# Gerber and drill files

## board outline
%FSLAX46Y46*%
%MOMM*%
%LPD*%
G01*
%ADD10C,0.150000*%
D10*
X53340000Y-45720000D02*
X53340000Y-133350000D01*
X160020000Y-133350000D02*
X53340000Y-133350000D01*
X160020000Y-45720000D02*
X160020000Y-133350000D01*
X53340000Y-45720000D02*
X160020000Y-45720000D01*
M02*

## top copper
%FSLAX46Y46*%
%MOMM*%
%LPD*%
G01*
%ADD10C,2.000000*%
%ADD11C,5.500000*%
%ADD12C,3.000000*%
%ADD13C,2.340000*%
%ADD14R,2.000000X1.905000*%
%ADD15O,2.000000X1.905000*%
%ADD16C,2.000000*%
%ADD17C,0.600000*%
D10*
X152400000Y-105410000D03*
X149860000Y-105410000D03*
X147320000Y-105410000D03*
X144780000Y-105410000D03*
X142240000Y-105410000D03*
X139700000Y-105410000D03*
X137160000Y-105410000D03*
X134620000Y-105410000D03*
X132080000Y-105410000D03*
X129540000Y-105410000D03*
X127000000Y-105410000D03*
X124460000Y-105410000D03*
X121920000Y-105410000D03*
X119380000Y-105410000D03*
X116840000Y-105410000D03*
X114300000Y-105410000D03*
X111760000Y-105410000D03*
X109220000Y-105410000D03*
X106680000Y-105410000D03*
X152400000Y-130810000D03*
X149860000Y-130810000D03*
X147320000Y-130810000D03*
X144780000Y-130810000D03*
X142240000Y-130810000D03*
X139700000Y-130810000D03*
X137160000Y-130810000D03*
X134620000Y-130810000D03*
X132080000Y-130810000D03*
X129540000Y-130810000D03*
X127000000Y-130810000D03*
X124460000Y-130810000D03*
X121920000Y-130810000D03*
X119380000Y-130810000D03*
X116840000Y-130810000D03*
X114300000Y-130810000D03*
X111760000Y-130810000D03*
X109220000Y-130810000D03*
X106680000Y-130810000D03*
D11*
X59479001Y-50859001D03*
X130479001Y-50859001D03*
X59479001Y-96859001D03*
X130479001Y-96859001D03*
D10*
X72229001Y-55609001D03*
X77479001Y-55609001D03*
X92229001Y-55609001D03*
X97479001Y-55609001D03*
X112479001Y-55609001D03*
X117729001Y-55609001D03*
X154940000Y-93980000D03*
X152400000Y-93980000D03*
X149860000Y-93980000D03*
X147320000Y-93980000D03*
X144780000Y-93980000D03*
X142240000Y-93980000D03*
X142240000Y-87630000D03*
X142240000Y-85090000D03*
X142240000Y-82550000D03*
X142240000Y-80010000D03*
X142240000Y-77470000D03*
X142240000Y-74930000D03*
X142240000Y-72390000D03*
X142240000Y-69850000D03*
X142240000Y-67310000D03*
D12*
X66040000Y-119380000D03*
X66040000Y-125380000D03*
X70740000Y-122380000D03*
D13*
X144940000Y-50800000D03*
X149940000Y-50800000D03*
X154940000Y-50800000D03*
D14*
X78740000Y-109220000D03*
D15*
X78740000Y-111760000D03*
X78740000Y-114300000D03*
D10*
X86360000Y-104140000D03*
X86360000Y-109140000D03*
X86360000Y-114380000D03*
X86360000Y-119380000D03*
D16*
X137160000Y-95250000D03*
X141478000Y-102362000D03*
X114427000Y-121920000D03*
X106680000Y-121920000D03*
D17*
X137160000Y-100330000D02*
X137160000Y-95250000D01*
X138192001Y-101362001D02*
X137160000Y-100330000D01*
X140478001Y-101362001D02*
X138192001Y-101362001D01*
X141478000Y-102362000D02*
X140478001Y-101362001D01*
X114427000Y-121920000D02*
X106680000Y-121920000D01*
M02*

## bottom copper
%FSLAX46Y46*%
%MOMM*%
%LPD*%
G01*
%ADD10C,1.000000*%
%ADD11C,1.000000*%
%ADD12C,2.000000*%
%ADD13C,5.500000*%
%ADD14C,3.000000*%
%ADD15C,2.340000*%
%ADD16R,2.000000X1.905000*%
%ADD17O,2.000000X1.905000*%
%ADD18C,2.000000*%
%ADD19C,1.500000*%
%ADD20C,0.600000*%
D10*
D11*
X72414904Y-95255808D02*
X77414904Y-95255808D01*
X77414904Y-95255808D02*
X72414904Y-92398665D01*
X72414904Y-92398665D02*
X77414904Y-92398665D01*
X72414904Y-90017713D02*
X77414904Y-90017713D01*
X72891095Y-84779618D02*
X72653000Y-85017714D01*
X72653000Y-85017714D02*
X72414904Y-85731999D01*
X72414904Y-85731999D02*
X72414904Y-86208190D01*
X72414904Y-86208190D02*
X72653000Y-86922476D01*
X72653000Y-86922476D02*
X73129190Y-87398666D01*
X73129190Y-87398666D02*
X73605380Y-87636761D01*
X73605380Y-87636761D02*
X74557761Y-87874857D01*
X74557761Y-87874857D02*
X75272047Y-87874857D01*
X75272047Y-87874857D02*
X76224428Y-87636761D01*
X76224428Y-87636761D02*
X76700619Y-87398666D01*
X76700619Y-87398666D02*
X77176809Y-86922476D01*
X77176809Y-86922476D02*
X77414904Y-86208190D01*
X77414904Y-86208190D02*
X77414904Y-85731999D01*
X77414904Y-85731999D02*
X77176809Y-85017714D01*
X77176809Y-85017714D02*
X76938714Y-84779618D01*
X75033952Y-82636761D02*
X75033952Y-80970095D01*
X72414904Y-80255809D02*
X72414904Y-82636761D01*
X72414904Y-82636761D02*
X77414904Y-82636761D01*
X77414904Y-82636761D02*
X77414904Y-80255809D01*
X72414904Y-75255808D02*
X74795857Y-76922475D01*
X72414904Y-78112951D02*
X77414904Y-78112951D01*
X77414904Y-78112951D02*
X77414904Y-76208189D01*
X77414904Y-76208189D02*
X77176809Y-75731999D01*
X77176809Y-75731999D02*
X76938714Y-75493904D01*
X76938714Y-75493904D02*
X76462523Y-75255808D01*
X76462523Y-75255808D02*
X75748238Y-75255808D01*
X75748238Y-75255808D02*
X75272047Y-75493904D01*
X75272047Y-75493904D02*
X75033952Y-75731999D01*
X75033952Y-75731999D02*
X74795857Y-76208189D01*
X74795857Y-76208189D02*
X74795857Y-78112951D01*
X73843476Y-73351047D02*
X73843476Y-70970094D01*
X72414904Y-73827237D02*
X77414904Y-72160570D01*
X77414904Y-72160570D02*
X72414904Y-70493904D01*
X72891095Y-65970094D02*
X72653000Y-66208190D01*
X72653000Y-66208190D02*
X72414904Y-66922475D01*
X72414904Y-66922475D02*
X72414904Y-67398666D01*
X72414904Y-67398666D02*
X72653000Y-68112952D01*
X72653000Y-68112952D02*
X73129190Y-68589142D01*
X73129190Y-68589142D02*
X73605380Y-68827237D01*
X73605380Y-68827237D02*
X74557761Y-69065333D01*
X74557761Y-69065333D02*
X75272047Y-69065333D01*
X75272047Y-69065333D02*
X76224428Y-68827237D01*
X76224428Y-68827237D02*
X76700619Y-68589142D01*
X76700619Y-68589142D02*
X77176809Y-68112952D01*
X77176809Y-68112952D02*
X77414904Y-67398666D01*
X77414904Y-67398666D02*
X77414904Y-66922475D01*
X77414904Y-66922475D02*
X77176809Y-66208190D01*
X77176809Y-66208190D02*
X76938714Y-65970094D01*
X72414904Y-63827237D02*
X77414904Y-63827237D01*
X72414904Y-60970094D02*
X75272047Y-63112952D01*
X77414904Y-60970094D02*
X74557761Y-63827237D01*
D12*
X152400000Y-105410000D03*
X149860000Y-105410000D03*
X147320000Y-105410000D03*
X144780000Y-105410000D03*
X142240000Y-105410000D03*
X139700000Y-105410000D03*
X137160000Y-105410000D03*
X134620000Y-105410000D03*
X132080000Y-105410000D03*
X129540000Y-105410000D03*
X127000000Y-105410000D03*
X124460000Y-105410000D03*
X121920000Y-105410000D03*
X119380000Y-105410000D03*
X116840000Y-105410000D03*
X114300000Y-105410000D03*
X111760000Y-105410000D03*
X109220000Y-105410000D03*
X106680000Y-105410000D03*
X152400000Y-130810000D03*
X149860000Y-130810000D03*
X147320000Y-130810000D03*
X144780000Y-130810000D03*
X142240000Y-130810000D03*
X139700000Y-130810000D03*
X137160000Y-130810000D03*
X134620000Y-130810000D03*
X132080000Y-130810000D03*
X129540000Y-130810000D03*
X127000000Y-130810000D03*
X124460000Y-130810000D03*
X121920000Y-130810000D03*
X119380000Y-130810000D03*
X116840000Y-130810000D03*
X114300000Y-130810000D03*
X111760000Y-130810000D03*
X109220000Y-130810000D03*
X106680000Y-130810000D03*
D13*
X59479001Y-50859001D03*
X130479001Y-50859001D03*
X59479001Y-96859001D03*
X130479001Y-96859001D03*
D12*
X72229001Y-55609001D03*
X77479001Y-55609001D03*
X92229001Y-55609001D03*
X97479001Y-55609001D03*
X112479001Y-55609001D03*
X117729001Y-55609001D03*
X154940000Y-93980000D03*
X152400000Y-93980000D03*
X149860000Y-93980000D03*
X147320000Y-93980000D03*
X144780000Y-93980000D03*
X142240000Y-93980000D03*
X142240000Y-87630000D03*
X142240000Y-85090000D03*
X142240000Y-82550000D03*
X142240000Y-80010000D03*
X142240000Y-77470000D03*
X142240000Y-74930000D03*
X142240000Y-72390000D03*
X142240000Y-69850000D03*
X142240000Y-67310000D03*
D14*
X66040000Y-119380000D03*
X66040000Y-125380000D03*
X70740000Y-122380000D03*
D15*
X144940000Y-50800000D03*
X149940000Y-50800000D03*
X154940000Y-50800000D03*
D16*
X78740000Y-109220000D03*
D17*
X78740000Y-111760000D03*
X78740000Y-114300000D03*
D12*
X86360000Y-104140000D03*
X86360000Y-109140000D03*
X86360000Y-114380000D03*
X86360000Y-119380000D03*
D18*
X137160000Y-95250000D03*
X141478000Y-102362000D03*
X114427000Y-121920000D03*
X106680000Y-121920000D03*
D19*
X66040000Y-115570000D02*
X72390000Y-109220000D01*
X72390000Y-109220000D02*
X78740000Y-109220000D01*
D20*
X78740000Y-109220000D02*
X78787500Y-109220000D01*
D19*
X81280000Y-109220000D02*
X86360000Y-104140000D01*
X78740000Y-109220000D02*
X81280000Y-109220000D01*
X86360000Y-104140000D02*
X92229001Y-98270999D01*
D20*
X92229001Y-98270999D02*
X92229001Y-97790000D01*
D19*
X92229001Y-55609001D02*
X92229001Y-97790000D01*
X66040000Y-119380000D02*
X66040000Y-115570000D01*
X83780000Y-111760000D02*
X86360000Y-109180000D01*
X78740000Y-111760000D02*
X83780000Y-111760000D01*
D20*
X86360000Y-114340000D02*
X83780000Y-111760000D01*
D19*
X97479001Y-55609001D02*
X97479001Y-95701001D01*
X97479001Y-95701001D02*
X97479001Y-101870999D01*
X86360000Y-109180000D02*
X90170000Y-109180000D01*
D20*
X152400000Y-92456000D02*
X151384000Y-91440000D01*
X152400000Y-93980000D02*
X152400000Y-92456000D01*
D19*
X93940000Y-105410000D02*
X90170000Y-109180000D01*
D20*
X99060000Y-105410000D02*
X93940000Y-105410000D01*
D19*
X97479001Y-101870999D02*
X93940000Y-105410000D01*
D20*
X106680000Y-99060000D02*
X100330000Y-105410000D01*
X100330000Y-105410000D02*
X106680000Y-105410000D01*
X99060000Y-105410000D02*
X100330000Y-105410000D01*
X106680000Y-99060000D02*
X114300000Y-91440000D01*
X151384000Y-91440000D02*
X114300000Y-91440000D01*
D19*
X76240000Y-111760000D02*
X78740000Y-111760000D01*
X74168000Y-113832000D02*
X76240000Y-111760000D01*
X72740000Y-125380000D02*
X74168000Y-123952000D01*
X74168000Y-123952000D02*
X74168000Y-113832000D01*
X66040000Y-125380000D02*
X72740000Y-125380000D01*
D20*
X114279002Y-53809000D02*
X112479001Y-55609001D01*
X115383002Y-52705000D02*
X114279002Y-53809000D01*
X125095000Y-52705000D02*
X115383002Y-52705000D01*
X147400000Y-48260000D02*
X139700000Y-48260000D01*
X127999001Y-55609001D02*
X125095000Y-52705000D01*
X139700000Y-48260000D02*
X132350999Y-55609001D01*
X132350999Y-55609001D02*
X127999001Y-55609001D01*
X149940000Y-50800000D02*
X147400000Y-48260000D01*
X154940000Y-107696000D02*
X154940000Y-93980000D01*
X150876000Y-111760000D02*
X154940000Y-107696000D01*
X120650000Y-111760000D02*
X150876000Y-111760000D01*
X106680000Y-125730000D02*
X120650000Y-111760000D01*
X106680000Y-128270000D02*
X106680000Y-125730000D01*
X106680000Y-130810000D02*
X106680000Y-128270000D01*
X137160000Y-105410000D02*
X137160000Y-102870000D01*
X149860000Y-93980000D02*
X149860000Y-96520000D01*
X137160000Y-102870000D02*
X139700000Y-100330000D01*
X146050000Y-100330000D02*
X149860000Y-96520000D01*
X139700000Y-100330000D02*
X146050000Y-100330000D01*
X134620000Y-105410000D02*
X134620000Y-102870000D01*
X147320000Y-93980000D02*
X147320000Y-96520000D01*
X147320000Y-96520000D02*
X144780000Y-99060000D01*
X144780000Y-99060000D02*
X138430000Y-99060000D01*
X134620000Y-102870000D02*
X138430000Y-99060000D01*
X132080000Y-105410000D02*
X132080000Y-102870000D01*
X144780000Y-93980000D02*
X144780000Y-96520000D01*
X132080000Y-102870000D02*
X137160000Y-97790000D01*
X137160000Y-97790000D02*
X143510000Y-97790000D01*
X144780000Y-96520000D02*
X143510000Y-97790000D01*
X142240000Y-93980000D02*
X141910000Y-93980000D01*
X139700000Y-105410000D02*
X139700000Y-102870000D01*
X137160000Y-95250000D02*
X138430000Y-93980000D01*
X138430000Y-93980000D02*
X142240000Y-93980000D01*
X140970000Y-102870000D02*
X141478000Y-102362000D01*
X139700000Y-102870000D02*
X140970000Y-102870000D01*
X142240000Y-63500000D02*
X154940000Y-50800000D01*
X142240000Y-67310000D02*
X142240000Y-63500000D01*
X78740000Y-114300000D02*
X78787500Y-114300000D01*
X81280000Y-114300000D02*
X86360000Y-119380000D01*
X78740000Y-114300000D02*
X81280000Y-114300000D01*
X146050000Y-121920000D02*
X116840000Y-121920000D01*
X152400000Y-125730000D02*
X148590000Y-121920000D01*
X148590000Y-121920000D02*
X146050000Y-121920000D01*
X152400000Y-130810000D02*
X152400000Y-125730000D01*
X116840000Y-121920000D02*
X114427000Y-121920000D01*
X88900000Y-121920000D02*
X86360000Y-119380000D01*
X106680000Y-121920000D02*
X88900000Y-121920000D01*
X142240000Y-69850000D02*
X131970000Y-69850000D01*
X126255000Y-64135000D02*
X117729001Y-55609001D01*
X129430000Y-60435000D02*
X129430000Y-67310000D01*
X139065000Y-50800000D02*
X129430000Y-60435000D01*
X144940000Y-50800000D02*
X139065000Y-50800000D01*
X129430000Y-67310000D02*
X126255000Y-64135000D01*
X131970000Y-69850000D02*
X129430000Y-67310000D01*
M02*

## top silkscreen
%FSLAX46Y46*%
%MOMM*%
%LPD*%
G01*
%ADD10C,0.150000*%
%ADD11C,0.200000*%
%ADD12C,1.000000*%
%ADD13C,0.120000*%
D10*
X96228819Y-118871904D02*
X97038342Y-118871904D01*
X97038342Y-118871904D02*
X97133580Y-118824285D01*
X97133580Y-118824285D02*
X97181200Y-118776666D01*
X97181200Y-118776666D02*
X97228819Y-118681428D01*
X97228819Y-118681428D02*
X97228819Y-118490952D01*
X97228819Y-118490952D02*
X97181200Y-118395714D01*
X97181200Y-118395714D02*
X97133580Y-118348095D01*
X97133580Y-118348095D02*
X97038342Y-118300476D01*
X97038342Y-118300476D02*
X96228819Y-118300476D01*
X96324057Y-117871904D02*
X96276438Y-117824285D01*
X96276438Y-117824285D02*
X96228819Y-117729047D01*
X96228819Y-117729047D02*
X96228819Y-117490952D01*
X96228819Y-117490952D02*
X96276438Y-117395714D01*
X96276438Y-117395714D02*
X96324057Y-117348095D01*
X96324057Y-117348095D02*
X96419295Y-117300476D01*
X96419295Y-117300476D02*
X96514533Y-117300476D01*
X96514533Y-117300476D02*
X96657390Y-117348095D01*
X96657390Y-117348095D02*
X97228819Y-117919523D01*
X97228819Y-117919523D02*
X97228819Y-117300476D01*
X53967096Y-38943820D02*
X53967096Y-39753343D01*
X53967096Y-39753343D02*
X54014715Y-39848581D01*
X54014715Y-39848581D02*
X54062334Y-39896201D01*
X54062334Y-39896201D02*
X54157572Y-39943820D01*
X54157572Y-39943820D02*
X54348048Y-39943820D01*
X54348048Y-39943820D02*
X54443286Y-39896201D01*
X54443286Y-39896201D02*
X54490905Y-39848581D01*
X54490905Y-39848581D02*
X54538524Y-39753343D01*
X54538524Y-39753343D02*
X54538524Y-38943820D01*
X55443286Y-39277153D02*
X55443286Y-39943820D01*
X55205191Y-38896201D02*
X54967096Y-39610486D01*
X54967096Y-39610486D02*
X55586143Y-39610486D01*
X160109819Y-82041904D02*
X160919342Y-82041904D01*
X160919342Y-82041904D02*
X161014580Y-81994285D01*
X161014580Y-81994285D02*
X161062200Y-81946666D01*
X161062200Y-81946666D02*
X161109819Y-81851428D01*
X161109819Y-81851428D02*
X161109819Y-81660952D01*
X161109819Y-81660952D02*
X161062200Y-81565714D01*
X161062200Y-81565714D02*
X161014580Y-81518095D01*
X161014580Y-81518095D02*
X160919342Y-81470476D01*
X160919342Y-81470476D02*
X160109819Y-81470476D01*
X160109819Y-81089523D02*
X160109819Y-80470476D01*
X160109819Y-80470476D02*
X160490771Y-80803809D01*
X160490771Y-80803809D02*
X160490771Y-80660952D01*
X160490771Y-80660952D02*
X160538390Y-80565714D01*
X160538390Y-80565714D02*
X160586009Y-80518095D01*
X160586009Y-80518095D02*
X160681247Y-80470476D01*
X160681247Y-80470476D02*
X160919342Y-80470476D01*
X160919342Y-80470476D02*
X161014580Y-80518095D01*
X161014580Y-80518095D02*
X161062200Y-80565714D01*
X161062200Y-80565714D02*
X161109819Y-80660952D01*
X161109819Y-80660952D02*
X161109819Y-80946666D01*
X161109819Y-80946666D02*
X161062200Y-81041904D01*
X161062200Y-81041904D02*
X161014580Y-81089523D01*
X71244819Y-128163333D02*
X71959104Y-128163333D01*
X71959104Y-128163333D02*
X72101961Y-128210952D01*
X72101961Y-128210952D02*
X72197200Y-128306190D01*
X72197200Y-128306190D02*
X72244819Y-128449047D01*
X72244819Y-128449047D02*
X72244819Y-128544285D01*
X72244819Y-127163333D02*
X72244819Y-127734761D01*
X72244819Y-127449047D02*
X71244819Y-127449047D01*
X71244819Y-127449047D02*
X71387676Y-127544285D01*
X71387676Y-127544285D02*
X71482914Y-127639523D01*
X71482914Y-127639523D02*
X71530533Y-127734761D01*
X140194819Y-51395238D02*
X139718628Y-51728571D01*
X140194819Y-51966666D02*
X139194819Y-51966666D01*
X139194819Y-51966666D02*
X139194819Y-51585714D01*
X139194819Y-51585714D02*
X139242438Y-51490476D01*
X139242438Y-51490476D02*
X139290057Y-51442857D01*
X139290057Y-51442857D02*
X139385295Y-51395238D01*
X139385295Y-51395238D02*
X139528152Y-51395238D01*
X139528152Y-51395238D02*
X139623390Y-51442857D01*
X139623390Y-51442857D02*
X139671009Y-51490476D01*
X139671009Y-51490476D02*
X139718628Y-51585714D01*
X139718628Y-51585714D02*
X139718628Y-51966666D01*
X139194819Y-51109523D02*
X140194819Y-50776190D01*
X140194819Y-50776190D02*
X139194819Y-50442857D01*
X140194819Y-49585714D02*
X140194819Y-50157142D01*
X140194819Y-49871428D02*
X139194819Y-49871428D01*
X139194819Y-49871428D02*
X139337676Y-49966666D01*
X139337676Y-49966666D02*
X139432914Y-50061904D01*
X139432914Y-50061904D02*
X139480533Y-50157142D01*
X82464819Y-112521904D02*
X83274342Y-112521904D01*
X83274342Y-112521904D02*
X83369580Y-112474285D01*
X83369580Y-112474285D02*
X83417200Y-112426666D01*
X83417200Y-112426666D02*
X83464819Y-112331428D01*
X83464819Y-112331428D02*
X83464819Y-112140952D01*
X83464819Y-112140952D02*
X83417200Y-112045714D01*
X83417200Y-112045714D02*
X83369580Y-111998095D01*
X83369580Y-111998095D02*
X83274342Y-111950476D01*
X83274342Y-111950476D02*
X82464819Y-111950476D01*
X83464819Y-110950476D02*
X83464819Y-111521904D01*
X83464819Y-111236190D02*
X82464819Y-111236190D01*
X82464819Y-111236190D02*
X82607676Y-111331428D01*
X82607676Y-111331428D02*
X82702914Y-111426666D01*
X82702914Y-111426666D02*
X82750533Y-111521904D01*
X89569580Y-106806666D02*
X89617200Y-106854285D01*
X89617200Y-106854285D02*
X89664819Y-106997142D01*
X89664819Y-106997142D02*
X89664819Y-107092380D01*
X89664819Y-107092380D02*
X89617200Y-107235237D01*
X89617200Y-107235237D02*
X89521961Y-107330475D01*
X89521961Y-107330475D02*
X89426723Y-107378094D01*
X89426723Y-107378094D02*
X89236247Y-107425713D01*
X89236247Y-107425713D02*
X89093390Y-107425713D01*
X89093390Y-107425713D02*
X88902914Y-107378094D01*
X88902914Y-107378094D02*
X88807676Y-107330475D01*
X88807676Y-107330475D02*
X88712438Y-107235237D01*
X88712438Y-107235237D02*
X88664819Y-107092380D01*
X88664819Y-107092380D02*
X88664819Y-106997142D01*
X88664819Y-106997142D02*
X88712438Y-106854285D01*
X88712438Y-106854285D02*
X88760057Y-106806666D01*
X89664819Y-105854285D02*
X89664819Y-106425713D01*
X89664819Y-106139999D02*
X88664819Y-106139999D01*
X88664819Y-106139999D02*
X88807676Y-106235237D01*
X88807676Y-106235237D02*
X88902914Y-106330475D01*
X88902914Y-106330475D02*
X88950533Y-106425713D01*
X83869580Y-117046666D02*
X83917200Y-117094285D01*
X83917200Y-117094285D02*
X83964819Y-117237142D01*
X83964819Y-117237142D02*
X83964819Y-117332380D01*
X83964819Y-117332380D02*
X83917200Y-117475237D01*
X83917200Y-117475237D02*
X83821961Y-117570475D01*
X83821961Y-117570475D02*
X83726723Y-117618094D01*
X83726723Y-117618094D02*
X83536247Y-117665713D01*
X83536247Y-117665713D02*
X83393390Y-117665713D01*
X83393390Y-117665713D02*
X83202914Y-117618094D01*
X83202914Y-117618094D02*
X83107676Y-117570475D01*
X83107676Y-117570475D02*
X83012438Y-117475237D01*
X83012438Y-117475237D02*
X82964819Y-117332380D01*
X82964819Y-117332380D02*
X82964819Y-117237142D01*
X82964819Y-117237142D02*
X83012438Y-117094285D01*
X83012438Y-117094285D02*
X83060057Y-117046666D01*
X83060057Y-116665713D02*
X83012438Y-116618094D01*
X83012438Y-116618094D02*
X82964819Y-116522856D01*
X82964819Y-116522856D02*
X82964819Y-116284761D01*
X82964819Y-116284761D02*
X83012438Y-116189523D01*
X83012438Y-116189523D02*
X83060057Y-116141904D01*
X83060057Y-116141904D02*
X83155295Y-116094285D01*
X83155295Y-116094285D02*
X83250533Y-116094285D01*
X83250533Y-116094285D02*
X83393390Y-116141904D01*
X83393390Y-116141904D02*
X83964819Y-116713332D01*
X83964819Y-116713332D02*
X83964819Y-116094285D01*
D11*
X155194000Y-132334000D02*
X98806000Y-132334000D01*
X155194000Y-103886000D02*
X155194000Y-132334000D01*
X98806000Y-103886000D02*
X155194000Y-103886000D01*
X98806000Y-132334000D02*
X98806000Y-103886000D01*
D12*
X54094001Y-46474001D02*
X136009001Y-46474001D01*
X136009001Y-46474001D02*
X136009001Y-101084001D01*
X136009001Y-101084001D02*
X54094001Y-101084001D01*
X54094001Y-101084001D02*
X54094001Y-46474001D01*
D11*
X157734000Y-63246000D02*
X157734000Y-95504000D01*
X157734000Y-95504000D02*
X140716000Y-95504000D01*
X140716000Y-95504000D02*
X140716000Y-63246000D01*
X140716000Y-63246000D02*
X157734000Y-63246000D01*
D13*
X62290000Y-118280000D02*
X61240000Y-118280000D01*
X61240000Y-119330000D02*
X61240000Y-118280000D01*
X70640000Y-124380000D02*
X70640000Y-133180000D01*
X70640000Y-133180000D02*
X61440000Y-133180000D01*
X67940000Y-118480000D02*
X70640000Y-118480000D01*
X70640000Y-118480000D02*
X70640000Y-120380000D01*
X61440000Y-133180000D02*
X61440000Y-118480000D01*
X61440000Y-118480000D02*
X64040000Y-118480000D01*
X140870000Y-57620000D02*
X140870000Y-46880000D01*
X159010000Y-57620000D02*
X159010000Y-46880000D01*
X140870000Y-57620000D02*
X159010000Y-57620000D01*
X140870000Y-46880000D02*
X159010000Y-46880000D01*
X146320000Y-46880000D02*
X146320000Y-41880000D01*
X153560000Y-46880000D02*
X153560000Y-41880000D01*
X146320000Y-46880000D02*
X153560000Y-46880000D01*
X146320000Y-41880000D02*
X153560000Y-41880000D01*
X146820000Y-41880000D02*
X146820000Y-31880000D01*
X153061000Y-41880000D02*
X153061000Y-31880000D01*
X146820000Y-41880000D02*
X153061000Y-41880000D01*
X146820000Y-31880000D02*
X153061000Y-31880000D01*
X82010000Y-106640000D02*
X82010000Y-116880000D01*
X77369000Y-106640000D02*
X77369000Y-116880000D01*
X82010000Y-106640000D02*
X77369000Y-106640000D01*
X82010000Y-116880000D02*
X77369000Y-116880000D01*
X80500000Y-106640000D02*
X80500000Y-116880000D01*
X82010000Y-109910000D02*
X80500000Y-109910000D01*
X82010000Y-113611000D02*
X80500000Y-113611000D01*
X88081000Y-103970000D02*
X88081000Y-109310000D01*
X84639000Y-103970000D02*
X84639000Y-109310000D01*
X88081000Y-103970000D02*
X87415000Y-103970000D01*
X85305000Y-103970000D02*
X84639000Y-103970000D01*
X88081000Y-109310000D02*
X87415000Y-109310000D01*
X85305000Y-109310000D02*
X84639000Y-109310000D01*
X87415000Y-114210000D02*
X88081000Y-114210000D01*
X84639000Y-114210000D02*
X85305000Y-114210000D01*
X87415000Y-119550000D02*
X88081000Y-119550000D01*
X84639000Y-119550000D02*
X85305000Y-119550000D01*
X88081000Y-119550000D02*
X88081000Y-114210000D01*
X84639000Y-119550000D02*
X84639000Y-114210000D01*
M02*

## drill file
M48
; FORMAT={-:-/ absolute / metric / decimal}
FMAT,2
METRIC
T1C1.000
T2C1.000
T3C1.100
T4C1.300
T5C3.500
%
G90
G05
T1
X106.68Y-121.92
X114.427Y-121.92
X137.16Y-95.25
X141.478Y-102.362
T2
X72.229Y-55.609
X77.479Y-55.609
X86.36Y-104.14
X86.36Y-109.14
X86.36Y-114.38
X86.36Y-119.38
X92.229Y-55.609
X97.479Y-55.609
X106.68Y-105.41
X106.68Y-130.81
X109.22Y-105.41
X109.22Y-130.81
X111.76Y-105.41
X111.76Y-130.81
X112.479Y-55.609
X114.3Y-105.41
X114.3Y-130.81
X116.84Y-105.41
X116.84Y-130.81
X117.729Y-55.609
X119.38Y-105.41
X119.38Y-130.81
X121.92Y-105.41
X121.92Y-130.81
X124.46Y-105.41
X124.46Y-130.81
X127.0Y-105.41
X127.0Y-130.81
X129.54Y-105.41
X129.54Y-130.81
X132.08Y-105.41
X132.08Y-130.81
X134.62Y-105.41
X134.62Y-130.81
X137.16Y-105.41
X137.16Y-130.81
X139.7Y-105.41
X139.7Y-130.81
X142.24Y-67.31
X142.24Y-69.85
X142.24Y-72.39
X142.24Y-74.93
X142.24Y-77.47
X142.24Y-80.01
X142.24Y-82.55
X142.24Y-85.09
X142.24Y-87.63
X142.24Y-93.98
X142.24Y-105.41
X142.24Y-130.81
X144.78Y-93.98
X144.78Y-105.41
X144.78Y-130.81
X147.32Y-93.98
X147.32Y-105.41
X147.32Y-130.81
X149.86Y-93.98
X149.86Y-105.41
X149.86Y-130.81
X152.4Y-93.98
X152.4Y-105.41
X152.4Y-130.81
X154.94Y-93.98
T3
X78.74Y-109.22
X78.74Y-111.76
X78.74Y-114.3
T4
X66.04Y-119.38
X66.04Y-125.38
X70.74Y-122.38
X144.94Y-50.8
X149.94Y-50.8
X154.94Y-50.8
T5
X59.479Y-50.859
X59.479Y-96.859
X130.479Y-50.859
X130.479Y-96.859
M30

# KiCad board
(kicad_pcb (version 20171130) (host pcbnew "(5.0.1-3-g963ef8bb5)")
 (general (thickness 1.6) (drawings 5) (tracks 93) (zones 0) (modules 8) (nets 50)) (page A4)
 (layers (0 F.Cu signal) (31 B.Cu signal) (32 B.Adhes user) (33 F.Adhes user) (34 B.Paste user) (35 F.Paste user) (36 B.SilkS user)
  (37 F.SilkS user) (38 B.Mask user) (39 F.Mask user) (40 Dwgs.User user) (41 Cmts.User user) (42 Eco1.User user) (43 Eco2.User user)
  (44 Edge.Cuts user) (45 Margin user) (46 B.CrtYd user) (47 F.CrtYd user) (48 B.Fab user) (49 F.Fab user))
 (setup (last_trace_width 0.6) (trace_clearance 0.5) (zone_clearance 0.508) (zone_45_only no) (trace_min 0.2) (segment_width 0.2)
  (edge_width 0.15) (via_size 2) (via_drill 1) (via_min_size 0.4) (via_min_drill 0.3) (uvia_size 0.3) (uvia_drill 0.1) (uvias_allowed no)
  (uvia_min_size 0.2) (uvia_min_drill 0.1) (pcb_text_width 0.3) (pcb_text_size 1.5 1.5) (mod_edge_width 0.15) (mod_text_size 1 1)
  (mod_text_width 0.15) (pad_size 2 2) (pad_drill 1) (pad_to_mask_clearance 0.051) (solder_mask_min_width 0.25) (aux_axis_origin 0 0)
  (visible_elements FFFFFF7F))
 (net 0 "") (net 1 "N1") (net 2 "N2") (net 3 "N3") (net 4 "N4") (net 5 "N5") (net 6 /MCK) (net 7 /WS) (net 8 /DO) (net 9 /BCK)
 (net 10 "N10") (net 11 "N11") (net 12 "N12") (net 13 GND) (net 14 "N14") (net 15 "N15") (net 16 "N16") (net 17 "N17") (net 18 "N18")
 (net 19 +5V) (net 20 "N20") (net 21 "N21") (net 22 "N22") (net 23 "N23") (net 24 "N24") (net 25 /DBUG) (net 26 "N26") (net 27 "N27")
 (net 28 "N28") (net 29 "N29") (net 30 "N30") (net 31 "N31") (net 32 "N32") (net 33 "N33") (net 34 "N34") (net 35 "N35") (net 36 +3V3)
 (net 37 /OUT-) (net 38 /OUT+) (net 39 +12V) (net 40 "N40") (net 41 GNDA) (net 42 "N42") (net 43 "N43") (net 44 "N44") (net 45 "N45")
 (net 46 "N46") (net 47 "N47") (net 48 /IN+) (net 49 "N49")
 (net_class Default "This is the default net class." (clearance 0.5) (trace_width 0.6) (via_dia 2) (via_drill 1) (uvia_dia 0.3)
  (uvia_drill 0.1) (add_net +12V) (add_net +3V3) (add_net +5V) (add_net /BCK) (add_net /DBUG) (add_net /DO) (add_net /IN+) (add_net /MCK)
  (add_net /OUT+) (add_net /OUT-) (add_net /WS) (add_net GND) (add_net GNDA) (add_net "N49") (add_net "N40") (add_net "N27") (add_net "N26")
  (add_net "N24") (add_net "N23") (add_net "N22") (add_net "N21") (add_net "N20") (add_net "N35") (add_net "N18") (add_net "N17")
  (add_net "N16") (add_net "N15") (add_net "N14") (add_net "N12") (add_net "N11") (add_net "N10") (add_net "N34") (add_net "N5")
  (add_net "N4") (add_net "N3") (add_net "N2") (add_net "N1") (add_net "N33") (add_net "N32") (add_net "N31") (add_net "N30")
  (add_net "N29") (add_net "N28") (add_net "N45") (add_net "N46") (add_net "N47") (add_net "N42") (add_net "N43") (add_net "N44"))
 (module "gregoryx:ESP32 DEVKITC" (layer F.Cu) (at 104.14 118.11 90)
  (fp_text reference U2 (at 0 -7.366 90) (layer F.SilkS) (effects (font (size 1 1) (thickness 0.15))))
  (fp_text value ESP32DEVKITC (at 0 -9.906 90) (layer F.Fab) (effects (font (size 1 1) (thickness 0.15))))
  (fp_line (start -14.224 51.054) (end -14.224 -5.334) (layer F.SilkS) (width 0.2))
  (fp_line (start 14.224 51.054) (end -14.224 51.054) (layer F.SilkS) (width 0.2))
  (fp_line (start 14.224 -5.334) (end 14.224 51.054) (layer F.SilkS) (width 0.2))
  (fp_line (start -14.224 -5.334) (end 14.224 -5.334) (layer F.SilkS) (width 0.2))
  (pad 38 thru_hole circle (at 12.7 48.26 90) (size 2 2) (drill 1) (layers *.Cu *.Mask) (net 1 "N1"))
  (pad 37 thru_hole circle (at 12.7 45.72 90) (size 2 2) (drill 1) (layers *.Cu *.Mask) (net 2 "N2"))
  (pad 36 thru_hole circle (at 12.7 43.18 90) (size 2 2) (drill 1) (layers *.Cu *.Mask) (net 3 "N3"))
  (pad 35 thru_hole circle (at 12.7 40.64 90) (size 2 2) (drill 1) (layers *.Cu *.Mask) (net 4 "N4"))
  (pad 34 thru_hole circle (at 12.7 38.1 90) (size 2 2) (drill 1) (layers *.Cu *.Mask) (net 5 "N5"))
  (pad 33 thru_hole circle (at 12.7 35.56 90) (size 2 2) (drill 1) (layers *.Cu *.Mask) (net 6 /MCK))
  (pad 32 thru_hole circle (at 12.7 33.02 90) (size 2 2) (drill 1) (layers *.Cu *.Mask) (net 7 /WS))
  (pad 31 thru_hole circle (at 12.7 30.48 90) (size 2 2) (drill 1) (layers *.Cu *.Mask) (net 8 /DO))
  (pad 30 thru_hole circle (at 12.7 27.94 90) (size 2 2) (drill 1) (layers *.Cu *.Mask) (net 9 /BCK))
  (pad 29 thru_hole circle (at 12.7 25.4 90) (size 2 2) (drill 1) (layers *.Cu *.Mask) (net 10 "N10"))
  (pad 28 thru_hole circle (at 12.7 22.86 90) (size 2 2) (drill 1) (layers *.Cu *.Mask) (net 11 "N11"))
  (pad 27 thru_hole circle (at 12.7 20.32 90) (size 2 2) (drill 1) (layers *.Cu *.Mask) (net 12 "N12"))
  (pad 26 thru_hole circle (at 12.7 17.78 90) (size 2 2) (drill 1) (layers *.Cu *.Mask) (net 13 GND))
  (pad 25 thru_hole circle (at 12.7 15.24 90) (size 2 2) (drill 1) (layers *.Cu *.Mask) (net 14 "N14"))
  (pad 24 thru_hole circle (at 12.7 12.7 90) (size 2 2) (drill 1) (layers *.Cu *.Mask) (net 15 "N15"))
  (pad 23 thru_hole circle (at 12.7 10.16 90) (size 2 2) (drill 1) (layers *.Cu *.Mask) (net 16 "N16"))
  (pad 22 thru_hole circle (at 12.7 7.62 90) (size 2 2) (drill 1) (layers *.Cu *.Mask) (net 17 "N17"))
  (pad 21 thru_hole circle (at 12.7 5.08 90) (size 2 2) (drill 1) (layers *.Cu *.Mask) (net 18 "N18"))
  (pad 20 thru_hole circle (at 12.7 2.54 90) (size 2 2) (drill 1) (layers *.Cu *.Mask) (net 13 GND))
  (pad 19 thru_hole circle (at -12.7 48.26 90) (size 2 2) (drill 1) (layers *.Cu *.Mask) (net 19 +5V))
  (pad 18 thru_hole circle (at -12.7 45.72 90) (size 2 2) (drill 1) (layers *.Cu *.Mask) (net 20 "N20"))
  (pad 17 thru_hole circle (at -12.7 43.18 90) (size 2 2) (drill 1) (layers *.Cu *.Mask) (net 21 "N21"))
  (pad 16 thru_hole circle (at -12.7 40.64 90) (size 2 2) (drill 1) (layers *.Cu *.Mask) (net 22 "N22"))
  (pad 15 thru_hole circle (at -12.7 38.1 90) (size 2 2) (drill 1) (layers *.Cu *.Mask) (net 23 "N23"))
  (pad 14 thru_hole circle (at -12.7 35.56 90) (size 2 2) (drill 1) (layers *.Cu *.Mask) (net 13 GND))
  (pad 13 thru_hole circle (at -12.7 33.02 90) (size 2 2) (drill 1) (layers *.Cu *.Mask) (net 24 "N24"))
  (pad 12 thru_hole circle (at -12.7 30.48 90) (size 2 2) (drill 1) (layers *.Cu *.Mask) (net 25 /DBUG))
  (pad 11 thru_hole circle (at -12.7 27.94 90) (size 2 2) (drill 1) (layers *.Cu *.Mask) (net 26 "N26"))
  (pad 10 thru_hole circle (at -12.7 25.4 90) (size 2 2) (drill 1) (layers *.Cu *.Mask) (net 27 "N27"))
  (pad 9 thru_hole circle (at -12.7 22.86 90) (size 2 2) (drill 1) (layers *.Cu *.Mask) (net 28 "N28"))
  (pad 8 thru_hole circle (at -12.7 20.32 90) (size 2 2) (drill 1) (layers *.Cu *.Mask) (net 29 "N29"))
  (pad 7 thru_hole circle (at -12.7 17.78 90) (size 2 2) (drill 1) (layers *.Cu *.Mask) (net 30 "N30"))
  (pad 6 thru_hole circle (at -12.7 15.24 90) (size 2 2) (drill 1) (layers *.Cu *.Mask) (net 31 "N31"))
  (pad 5 thru_hole circle (at -12.7 12.7 90) (size 2 2) (drill 1) (layers *.Cu *.Mask) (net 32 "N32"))
  (pad 4 thru_hole circle (at -12.7 10.16 90) (size 2 2) (drill 1) (layers *.Cu *.Mask) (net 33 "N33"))
  (pad 3 thru_hole circle (at -12.7 7.62 90) (size 2 2) (drill 1) (layers *.Cu *.Mask) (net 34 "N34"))
  (pad 2 thru_hole circle (at -12.7 5.08 90) (size 2 2) (drill 1) (layers *.Cu *.Mask) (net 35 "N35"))
  (pad 1 thru_hole circle (at -12.7 2.54 90) (size 2 2) (drill 1) (layers *.Cu *.Mask) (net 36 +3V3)))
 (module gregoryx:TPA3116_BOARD (layer F.Cu) (at 54.729001 47.109001)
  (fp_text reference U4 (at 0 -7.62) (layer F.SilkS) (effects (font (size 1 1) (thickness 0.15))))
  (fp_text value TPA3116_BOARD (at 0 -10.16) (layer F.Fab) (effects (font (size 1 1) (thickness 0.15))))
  (fp_line (start -0.635 -0.635) (end 81.28 -0.635) (layer F.SilkS) (width 1))
  (fp_line (start 81.28 -0.635) (end 81.28 53.975) (layer F.SilkS) (width 1))
  (fp_line (start 81.28 53.975) (end -0.635 53.975) (layer F.SilkS) (width 1))
  (fp_line (start -0.635 53.975) (end -0.635 -0.635) (layer F.SilkS) (width 1))
  (pad "" thru_hole circle (at 4.75 3.75) (size 5.5 5.5) (drill 3.5) (layers *.Cu *.Mask))
  (pad "" thru_hole circle (at 75.75 3.75) (size 5.5 5.5) (drill 3.5) (layers *.Cu *.Mask))
  (pad "" thru_hole circle (at 4.75 49.75) (size 5.5 5.5) (drill 3.5) (layers *.Cu *.Mask))
  (pad "" thru_hole circle (at 75.75 49.75) (size 5.5 5.5) (drill 3.5) (layers *.Cu *.Mask))
  (pad 6 thru_hole circle (at 17.5 8.5) (size 2 2) (drill 1) (layers *.Cu *.Mask) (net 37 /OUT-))
  (pad 5 thru_hole circle (at 22.75 8.5) (size 2 2) (drill 1) (layers *.Cu *.Mask) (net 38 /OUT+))
  (pad 4 thru_hole circle (at 37.5 8.5) (size 2 2) (drill 1) (layers *.Cu *.Mask) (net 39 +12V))
  (pad 3 thru_hole circle (at 42.75 8.5) (size 2 2) (drill 1) (layers *.Cu *.Mask) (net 13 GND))
  (pad 2 thru_hole circle (at 57.75 8.5) (size 2 2) (drill 1) (layers *.Cu *.Mask) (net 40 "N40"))
  (pad 1 thru_hole circle (at 63 8.5) (size 2 2) (drill 1) (layers *.Cu *.Mask) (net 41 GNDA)))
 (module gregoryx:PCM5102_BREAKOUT (layer F.Cu) (at 157.48 81.28 270)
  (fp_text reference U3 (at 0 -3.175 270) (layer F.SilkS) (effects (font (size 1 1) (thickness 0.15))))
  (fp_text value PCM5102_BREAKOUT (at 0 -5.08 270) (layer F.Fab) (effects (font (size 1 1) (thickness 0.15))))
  (fp_line (start -18.034 -0.254) (end 14.224 -0.254) (layer F.SilkS) (width 0.2))
  (fp_line (start 14.224 -0.254) (end 14.224 16.764) (layer F.SilkS) (width 0.2))
  (fp_line (start 14.224 16.764) (end -18.034 16.764) (layer F.SilkS) (width 0.2))
  (fp_line (start -18.034 16.764) (end -18.034 -0.254) (layer F.SilkS) (width 0.2))
  (pad 1 thru_hole circle (at 12.7 2.54 270) (size 2 2) (drill 1) (layers *.Cu *.Mask) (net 36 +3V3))
  (pad 2 thru_hole circle (at 12.7 5.08 270) (size 2 2) (drill 1) (layers *.Cu *.Mask) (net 13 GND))
  (pad 3 thru_hole circle (at 12.7 7.62 270) (size 2 2) (drill 1) (layers *.Cu *.Mask) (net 7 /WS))
  (pad 4 thru_hole circle (at 12.7 10.16 270) (size 2 2) (drill 1) (layers *.Cu *.Mask) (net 8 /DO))
  (pad 5 thru_hole circle (at 12.7 12.7 270) (size 2 2) (drill 1) (layers *.Cu *.Mask) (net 9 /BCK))
  (pad 6 thru_hole circle (at 12.7 15.24 270) (size 2 2) (drill 1) (layers *.Cu *.Mask) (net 6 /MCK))
  (pad 7 thru_hole circle (at 6.35 15.24 270) (size 2 2) (drill 1) (layers *.Cu *.Mask) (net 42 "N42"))
  (pad 8 thru_hole circle (at 3.81 15.24 270) (size 2 2) (drill 1) (layers *.Cu *.Mask) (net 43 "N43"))
  (pad 9 thru_hole circle (at 1.27 15.24 270) (size 2 2) (drill 1) (layers *.Cu *.Mask) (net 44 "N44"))
  (pad 10 thru_hole circle (at -1.27 15.24 270) (size 2 2) (drill 1) (layers *.Cu *.Mask) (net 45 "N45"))
  (pad "" thru_hole circle (at -3.81 15.24 270) (size 2 2) (drill 1) (layers *.Cu *.Mask))
  (pad 11 thru_hole circle (at -6.35 15.24 270) (size 2 2) (drill 1) (layers *.Cu *.Mask) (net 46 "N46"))
  (pad 12 thru_hole circle (at -8.89 15.24 270) (size 2 2) (drill 1) (layers *.Cu *.Mask) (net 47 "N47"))
  (pad 13 thru_hole circle (at -11.43 15.24 270) (size 2 2) (drill 1) (layers *.Cu *.Mask) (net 41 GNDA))
  (pad 14 thru_hole circle (at -13.97 15.24 270) (size 2 2) (drill 1) (layers *.Cu *.Mask) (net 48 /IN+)))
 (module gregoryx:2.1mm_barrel (layer F.Cu) (at 66.04 119.38 90)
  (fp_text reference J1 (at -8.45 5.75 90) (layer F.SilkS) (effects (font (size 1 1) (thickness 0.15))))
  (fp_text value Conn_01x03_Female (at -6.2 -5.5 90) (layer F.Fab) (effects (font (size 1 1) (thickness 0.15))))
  (fp_line (start 1.1 -3.75) (end 1.1 -4.8) (layer F.SilkS) (width 0.12))
  (fp_line (start 0.05 -4.8) (end 1.1 -4.8) (layer F.SilkS) (width 0.12))
  (fp_line (start -5 4.6) (end -13.8 4.6) (layer F.SilkS) (width 0.12))
  (fp_line (start -13.8 4.6) (end -13.8 -4.6) (layer F.SilkS) (width 0.12))
  (fp_line (start 0.9 1.9) (end 0.9 4.6) (layer F.SilkS) (width 0.12))
  (fp_line (start 0.9 4.6) (end -1 4.6) (layer F.SilkS) (width 0.12))
  (fp_line (start -13.8 -4.6) (end 0.9 -4.6) (layer F.SilkS) (width 0.12))
  (fp_line (start 0.9 -4.6) (end 0.9 -2) (layer F.SilkS) (width 0.12))
  (pad 1 thru_hole circle (at 0 0 90) (size 3 3) (drill 1.3) (layers *.Cu *.Mask) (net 39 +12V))
  (pad 2 thru_hole circle (at -6 0 90) (size 3 3) (drill 1.3) (layers *.Cu *.Mask) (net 13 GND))
  (pad 3 thru_hole circle (at -3 4.7 90) (size 3 3) (drill 1.3) (layers *.Cu *.Mask) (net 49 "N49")))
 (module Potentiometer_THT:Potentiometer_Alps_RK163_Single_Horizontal (layer F.Cu) (at 154.94 50.8 90)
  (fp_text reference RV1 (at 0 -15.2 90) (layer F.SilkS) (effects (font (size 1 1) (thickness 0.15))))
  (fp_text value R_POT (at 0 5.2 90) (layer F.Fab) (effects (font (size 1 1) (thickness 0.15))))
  (fp_line (start -6.82 -14.07) (end 3.92 -14.07) (layer F.SilkS) (width 0.12))
  (fp_line (start -6.82 4.07) (end 3.92 4.07) (layer F.SilkS) (width 0.12))
  (fp_line (start -6.82 -14.07) (end -6.82 4.07) (layer F.SilkS) (width 0.12))
  (fp_line (start 3.92 -14.07) (end 3.92 4.07) (layer F.SilkS) (width 0.12))
  (fp_line (start 3.92 -8.62) (end 8.92 -8.62) (layer F.SilkS) (width 0.12))
  (fp_line (start 3.92 -1.38) (end 8.92 -1.38) (layer F.SilkS) (width 0.12))
  (fp_line (start 3.92 -8.62) (end 3.92 -1.38) (layer F.SilkS) (width 0.12))
  (fp_line (start 8.92 -8.62) (end 8.92 -1.38) (layer F.SilkS) (width 0.12))
  (fp_line (start 8.92 -8.12) (end 18.92 -8.12) (layer F.SilkS) (width 0.12))
  (fp_line (start 8.92 -1.879) (end 18.92 -1.879) (layer F.SilkS) (width 0.12))
  (fp_line (start 8.92 -8.12) (end 8.92 -1.879) (layer F.SilkS) (width 0.12))
  (fp_line (start 18.92 -8.12) (end 18.92 -1.879) (layer F.SilkS) (width 0.12))
  (pad 3 thru_hole circle (at 0 -10 90) (size 2.34 2.34) (drill 1.3) (layers *.Cu *.Mask) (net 41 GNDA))
  (pad 2 thru_hole circle (at 0 -5 90) (size 2.34 2.34) (drill 1.3) (layers *.Cu *.Mask) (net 40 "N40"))
  (pad 1 thru_hole circle (at 0 0 90) (size 2.34 2.34) (drill 1.3) (layers *.Cu *.Mask) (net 48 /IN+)))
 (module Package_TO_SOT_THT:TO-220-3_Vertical (layer F.Cu) (at 78.74 109.22 270)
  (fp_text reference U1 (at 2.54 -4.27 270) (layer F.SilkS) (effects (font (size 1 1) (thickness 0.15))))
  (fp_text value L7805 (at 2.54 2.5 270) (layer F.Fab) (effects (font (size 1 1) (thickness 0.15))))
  (fp_line (start -2.58 -3.27) (end 7.66 -3.27) (layer F.SilkS) (width 0.12))
  (fp_line (start -2.58 1.371) (end 7.66 1.371) (layer F.SilkS) (width 0.12))
  (fp_line (start -2.58 -3.27) (end -2.58 1.371) (layer F.SilkS) (width 0.12))
  (fp_line (start 7.66 -3.27) (end 7.66 1.371) (layer F.SilkS) (width 0.12))
  (fp_line (start -2.58 -1.76) (end 7.66 -1.76) (layer F.SilkS) (width 0.12))
  (fp_line (start 0.69 -3.27) (end 0.69 -1.76) (layer F.SilkS) (width 0.12))
  (fp_line (start 4.391 -3.27) (end 4.391 -1.76) (layer F.SilkS) (width 0.12))
  (pad 1 thru_hole rect (at 0 0 270) (size 1.905 2) (drill 1.1) (layers *.Cu *.Mask) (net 39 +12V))
  (pad 2 thru_hole oval (at 2.54 0 270) (size 1.905 2) (drill 1.1) (layers *.Cu *.Mask) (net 13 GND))
  (pad 3 thru_hole oval (at 5.08 0 270) (size 1.905 2) (drill 1.1) (layers *.Cu *.Mask) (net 19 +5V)))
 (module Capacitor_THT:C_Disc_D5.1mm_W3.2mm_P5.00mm (layer F.Cu) (at 86.36 104.14 270)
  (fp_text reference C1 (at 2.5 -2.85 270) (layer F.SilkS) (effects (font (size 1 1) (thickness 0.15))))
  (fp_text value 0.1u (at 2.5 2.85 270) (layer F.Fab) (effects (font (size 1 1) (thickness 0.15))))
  (fp_line (start -0.17 -1.721) (end 5.17 -1.721) (layer F.SilkS) (width 0.12))
  (fp_line (start -0.17 1.721) (end 5.17 1.721) (layer F.SilkS) (width 0.12))
  (fp_line (start -0.17 -1.721) (end -0.17 -1.055) (layer F.SilkS) (width 0.12))
  (fp_line (start -0.17 1.055) (end -0.17 1.721) (layer F.SilkS) (width 0.12))
  (fp_line (start 5.17 -1.721) (end 5.17 -1.055) (layer F.SilkS) (width 0.12))
  (fp_line (start 5.17 1.055) (end 5.17 1.721) (layer F.SilkS) (width 0.12))
  (pad 1 thru_hole circle (at 0 0 270) (size 2 2) (drill 1) (layers *.Cu *.Mask) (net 39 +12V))
  (pad 2 thru_hole circle (at 5 0 270) (size 2 2) (drill 1) (layers *.Cu *.Mask) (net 13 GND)))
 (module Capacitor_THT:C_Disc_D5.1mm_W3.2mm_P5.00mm (layer F.Cu) (at 86.36 119.38 90)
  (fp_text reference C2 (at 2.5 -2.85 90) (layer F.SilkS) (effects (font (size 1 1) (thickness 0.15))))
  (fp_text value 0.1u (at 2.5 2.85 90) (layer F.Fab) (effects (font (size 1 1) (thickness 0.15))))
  (fp_line (start 5.17 1.055) (end 5.17 1.721) (layer F.SilkS) (width 0.12))
  (fp_line (start 5.17 -1.721) (end 5.17 -1.055) (layer F.SilkS) (width 0.12))
  (fp_line (start -0.17 1.055) (end -0.17 1.721) (layer F.SilkS) (width 0.12))
  (fp_line (start -0.17 -1.721) (end -0.17 -1.055) (layer F.SilkS) (width 0.12))
  (fp_line (start -0.17 1.721) (end 5.17 1.721) (layer F.SilkS) (width 0.12))
  (fp_line (start -0.17 -1.721) (end 5.17 -1.721) (layer F.SilkS) (width 0.12))
  (pad 2 thru_hole circle (at 5 0 90) (size 2 2) (drill 1) (layers *.Cu *.Mask) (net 13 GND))
  (pad 1 thru_hole circle (at 0 0 90) (size 2 2) (drill 1) (layers *.Cu *.Mask) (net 19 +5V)))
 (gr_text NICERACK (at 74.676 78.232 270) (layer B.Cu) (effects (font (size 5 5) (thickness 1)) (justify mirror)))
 (gr_line (start 53.34 45.72) (end 53.34 133.35) (layer Edge.Cuts) (width 0.15))
 (gr_line (start 160.02 133.35) (end 53.34 133.35) (layer Edge.Cuts) (width 0.15))
 (gr_line (start 160.02 45.72) (end 160.02 133.35) (layer Edge.Cuts) (width 0.15))
 (gr_line (start 53.34 45.72) (end 160.02 45.72) (layer Edge.Cuts) (width 0.15))
 (segment (start 66.04 115.57) (end 72.39 109.22) (width 1.5) (layer B.Cu) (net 39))
 (segment (start 72.39 109.22) (end 78.74 109.22) (width 1.5) (layer B.Cu) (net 39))
 (segment (start 78.74 109.22) (end 78.7875 109.22) (width 0.6) (layer B.Cu) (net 39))
 (segment (start 81.28 109.22) (end 86.36 104.14) (width 1.5) (layer B.Cu) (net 39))
 (segment (start 78.74 109.22) (end 81.28 109.22) (width 1.5) (layer B.Cu) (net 39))
 (segment (start 86.36 104.14) (end 92.229001 98.270999) (width 1.5) (layer B.Cu) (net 39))
 (segment (start 92.229001 98.270999) (end 92.229001 97.79) (width 0.6) (layer B.Cu) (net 39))
 (segment (start 92.229001 55.609001) (end 92.229001 97.79) (width 1.5) (layer B.Cu) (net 39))
 (segment (start 66.04 119.38) (end 66.04 115.57) (width 1.5) (layer B.Cu) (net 39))
 (segment (start 83.78 111.76) (end 86.36 109.18) (width 1.5) (layer B.Cu) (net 13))
 (segment (start 78.74 111.76) (end 83.78 111.76) (width 1.5) (layer B.Cu) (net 13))
 (segment (start 86.36 114.34) (end 83.78 111.76) (width 0.6) (layer B.Cu) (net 13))
 (segment (start 97.479001 55.609001) (end 97.479001 95.701001) (width 1.5) (layer B.Cu) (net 13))
 (segment (start 97.479001 95.701001) (end 97.479001 101.870999) (width 1.5) (layer B.Cu) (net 13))
 (segment (start 86.36 109.18) (end 90.17 109.18) (width 1.5) (layer B.Cu) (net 13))
 (segment (start 152.4 92.456) (end 151.384 91.44) (width 0.6) (layer B.Cu) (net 13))
 (segment (start 152.4 93.98) (end 152.4 92.456) (width 0.6) (layer B.Cu) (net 13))
 (segment (start 93.94 105.41) (end 90.17 109.18) (width 1.5) (layer B.Cu) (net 13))
 (segment (start 99.06 105.41) (end 93.94 105.41) (width 0.6) (layer B.Cu) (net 13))
 (segment (start 97.479001 101.870999) (end 93.94 105.41) (width 1.5) (layer B.Cu) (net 13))
 (segment (start 106.68 99.06) (end 100.33 105.41) (width 0.6) (layer B.Cu) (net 13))
 (segment (start 100.33 105.41) (end 106.68 105.41) (width 0.6) (layer B.Cu) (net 13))
 (segment (start 99.06 105.41) (end 100.33 105.41) (width 0.6) (layer B.Cu) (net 13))
 (segment (start 106.68 99.06) (end 114.3 91.44) (width 0.6) (layer B.Cu) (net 13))
 (segment (start 151.384 91.44) (end 114.3 91.44) (width 0.6) (layer B.Cu) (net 13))
 (segment (start 76.24 111.76) (end 78.74 111.76) (width 1.5) (layer B.Cu) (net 13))
 (segment (start 74.168 113.832) (end 76.24 111.76) (width 1.5) (layer B.Cu) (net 13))
 (segment (start 72.74 125.38) (end 74.168 123.952) (width 1.5) (layer B.Cu) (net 13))
 (segment (start 74.168 123.952) (end 74.168 113.832) (width 1.5) (layer B.Cu) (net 13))
 (segment (start 66.04 125.38) (end 72.74 125.38) (width 1.5) (layer B.Cu) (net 13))
 (segment (start 114.279002 53.809) (end 112.479001 55.609001) (width 0.6) (layer B.Cu) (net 40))
 (segment (start 115.383002 52.705) (end 114.279002 53.809) (width 0.6) (layer B.Cu) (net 40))
 (segment (start 125.095 52.705) (end 115.383002 52.705) (width 0.6) (layer B.Cu) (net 40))
 (segment (start 147.4 48.26) (end 139.7 48.26) (width 0.6) (layer B.Cu) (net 40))
 (segment (start 127.999001 55.609001) (end 125.095 52.705) (width 0.6) (layer B.Cu) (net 40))
 (segment (start 139.7 48.26) (end 132.350999 55.609001) (width 0.6) (layer B.Cu) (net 40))
 (segment (start 132.350999 55.609001) (end 127.999001 55.609001) (width 0.6) (layer B.Cu) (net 40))
 (segment (start 149.94 50.8) (end 147.4 48.26) (width 0.6) (layer B.Cu) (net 40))
 (segment (start 154.94 107.696) (end 154.94 93.98) (width 0.6) (layer B.Cu) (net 36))
 (segment (start 150.876 111.76) (end 154.94 107.696) (width 0.6) (layer B.Cu) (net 36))
 (segment (start 120.65 111.76) (end 150.876 111.76) (width 0.6) (layer B.Cu) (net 36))
 (segment (start 106.68 125.73) (end 120.65 111.76) (width 0.6) (layer B.Cu) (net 36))
 (segment (start 106.68 128.27) (end 106.68 125.73) (width 0.6) (layer B.Cu) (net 36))
 (segment (start 106.68 130.81) (end 106.68 128.27) (width 0.6) (layer B.Cu) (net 36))
 (segment (start 137.16 105.41) (end 137.16 102.87) (width 0.6) (layer B.Cu) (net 7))
 (segment (start 149.86 93.98) (end 149.86 96.52) (width 0.6) (layer B.Cu) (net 7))
 (segment (start 137.16 102.87) (end 139.7 100.33) (width 0.6) (layer B.Cu) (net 7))
 (segment (start 146.05 100.33) (end 149.86 96.52) (width 0.6) (layer B.Cu) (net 7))
 (segment (start 139.7 100.33) (end 146.05 100.33) (width 0.6) (layer B.Cu) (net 7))
 (segment (start 134.62 105.41) (end 134.62 102.87) (width 0.6) (layer B.Cu) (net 8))
 (segment (start 147.32 93.98) (end 147.32 96.52) (width 0.6) (layer B.Cu) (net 8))
 (segment (start 147.32 96.52) (end 144.78 99.06) (width 0.6) (layer B.Cu) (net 8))
 (segment (start 144.78 99.06) (end 138.43 99.06) (width 0.6) (layer B.Cu) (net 8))
 (segment (start 134.62 102.87) (end 138.43 99.06) (width 0.6) (layer B.Cu) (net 8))
 (segment (start 132.08 105.41) (end 132.08 102.87) (width 0.6) (layer B.Cu) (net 9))
 (segment (start 144.78 93.98) (end 144.78 96.52) (width 0.6) (layer B.Cu) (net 9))
 (segment (start 132.08 102.87) (end 137.16 97.79) (width 0.6) (layer B.Cu) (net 9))
 (segment (start 137.16 97.79) (end 143.51 97.79) (width 0.6) (layer B.Cu) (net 9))
 (segment (start 144.78 96.52) (end 143.51 97.79) (width 0.6) (layer B.Cu) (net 9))
 (segment (start 142.24 93.98) (end 141.91 93.98) (width 0.6) (layer B.Cu) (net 6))
 (segment (start 139.7 105.41) (end 139.7 102.87) (width 0.6) (layer B.Cu) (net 6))
 (via (at 137.16 95.25) (size 2) (drill 1) (layers F.Cu B.Cu) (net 6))
 (segment (start 137.16 100.33) (end 137.16 95.25) (width 0.6) (layer F.Cu) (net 6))
 (segment (start 137.16 95.25) (end 138.43 93.98) (width 0.6) (layer B.Cu) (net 6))
 (segment (start 138.43 93.98) (end 142.24 93.98) (width 0.6) (layer B.Cu) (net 6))
 (via (at 141.478 102.362) (size 2) (drill 1) (layers F.Cu B.Cu) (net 6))
 (segment (start 140.97 102.87) (end 141.478 102.362) (width 0.6) (layer B.Cu) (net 6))
 (segment (start 139.7 102.87) (end 140.97 102.87) (width 0.6) (layer B.Cu) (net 6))
 (segment (start 138.192001 101.362001) (end 137.16 100.33) (width 0.6) (layer F.Cu) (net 6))
 (segment (start 140.478001 101.362001) (end 138.192001 101.362001) (width 0.6) (layer F.Cu) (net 6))
 (segment (start 141.478 102.362) (end 140.478001 101.362001) (width 0.6) (layer F.Cu) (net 6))
 (segment (start 142.24 63.5) (end 154.94 50.8) (width 0.6) (layer B.Cu) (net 48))
 (segment (start 142.24 67.31) (end 142.24 63.5) (width 0.6) (layer B.Cu) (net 48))
 (segment (start 78.74 114.3) (end 78.7875 114.3) (width 0.6) (layer B.Cu) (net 19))
 (segment (start 81.28 114.3) (end 86.36 119.38) (width 0.6) (layer B.Cu) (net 19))
 (segment (start 78.74 114.3) (end 81.28 114.3) (width 0.6) (layer B.Cu) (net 19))
 (segment (start 146.05 121.92) (end 116.84 121.92) (width 0.6) (layer B.Cu) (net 19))
 (segment (start 152.4 125.73) (end 148.59 121.92) (width 0.6) (layer B.Cu) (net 19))
 (segment (start 148.59 121.92) (end 146.05 121.92) (width 0.6) (layer B.Cu) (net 19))
 (segment (start 152.4 130.81) (end 152.4 125.73) (width 0.6) (layer B.Cu) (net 19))
 (via (at 114.427 121.92) (size 2) (drill 1) (layers F.Cu B.Cu) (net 19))
 (segment (start 116.84 121.92) (end 114.427 121.92) (width 0.6) (layer B.Cu) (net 19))
 (via (at 106.68 121.92) (size 2) (drill 1) (layers F.Cu B.Cu) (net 19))
 (segment (start 114.427 121.92) (end 106.68 121.92) (width 0.6) (layer F.Cu) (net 19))
 (segment (start 88.9 121.92) (end 86.36 119.38) (width 0.6) (layer B.Cu) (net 19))
 (segment (start 106.68 121.92) (end 88.9 121.92) (width 0.6) (layer B.Cu) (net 19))
 (segment (start 142.24 69.85) (end 131.97 69.85) (width 0.6) (layer B.Cu) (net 41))
 (segment (start 126.255 64.135) (end 117.729001 55.609001) (width 0.6) (layer B.Cu) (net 41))
 (segment (start 129.43 60.435) (end 129.43 67.31) (width 0.6) (layer B.Cu) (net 41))
 (segment (start 139.065 50.8) (end 129.43 60.435) (width 0.6) (layer B.Cu) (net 41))
 (segment (start 144.94 50.8) (end 139.065 50.8) (width 0.6) (layer B.Cu) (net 41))
 (segment (start 129.43 67.31) (end 126.255 64.135) (width 0.6) (layer B.Cu) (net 41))
 (segment (start 131.97 69.85) (end 129.43 67.31) (width 0.6) (layer B.Cu) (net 41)))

